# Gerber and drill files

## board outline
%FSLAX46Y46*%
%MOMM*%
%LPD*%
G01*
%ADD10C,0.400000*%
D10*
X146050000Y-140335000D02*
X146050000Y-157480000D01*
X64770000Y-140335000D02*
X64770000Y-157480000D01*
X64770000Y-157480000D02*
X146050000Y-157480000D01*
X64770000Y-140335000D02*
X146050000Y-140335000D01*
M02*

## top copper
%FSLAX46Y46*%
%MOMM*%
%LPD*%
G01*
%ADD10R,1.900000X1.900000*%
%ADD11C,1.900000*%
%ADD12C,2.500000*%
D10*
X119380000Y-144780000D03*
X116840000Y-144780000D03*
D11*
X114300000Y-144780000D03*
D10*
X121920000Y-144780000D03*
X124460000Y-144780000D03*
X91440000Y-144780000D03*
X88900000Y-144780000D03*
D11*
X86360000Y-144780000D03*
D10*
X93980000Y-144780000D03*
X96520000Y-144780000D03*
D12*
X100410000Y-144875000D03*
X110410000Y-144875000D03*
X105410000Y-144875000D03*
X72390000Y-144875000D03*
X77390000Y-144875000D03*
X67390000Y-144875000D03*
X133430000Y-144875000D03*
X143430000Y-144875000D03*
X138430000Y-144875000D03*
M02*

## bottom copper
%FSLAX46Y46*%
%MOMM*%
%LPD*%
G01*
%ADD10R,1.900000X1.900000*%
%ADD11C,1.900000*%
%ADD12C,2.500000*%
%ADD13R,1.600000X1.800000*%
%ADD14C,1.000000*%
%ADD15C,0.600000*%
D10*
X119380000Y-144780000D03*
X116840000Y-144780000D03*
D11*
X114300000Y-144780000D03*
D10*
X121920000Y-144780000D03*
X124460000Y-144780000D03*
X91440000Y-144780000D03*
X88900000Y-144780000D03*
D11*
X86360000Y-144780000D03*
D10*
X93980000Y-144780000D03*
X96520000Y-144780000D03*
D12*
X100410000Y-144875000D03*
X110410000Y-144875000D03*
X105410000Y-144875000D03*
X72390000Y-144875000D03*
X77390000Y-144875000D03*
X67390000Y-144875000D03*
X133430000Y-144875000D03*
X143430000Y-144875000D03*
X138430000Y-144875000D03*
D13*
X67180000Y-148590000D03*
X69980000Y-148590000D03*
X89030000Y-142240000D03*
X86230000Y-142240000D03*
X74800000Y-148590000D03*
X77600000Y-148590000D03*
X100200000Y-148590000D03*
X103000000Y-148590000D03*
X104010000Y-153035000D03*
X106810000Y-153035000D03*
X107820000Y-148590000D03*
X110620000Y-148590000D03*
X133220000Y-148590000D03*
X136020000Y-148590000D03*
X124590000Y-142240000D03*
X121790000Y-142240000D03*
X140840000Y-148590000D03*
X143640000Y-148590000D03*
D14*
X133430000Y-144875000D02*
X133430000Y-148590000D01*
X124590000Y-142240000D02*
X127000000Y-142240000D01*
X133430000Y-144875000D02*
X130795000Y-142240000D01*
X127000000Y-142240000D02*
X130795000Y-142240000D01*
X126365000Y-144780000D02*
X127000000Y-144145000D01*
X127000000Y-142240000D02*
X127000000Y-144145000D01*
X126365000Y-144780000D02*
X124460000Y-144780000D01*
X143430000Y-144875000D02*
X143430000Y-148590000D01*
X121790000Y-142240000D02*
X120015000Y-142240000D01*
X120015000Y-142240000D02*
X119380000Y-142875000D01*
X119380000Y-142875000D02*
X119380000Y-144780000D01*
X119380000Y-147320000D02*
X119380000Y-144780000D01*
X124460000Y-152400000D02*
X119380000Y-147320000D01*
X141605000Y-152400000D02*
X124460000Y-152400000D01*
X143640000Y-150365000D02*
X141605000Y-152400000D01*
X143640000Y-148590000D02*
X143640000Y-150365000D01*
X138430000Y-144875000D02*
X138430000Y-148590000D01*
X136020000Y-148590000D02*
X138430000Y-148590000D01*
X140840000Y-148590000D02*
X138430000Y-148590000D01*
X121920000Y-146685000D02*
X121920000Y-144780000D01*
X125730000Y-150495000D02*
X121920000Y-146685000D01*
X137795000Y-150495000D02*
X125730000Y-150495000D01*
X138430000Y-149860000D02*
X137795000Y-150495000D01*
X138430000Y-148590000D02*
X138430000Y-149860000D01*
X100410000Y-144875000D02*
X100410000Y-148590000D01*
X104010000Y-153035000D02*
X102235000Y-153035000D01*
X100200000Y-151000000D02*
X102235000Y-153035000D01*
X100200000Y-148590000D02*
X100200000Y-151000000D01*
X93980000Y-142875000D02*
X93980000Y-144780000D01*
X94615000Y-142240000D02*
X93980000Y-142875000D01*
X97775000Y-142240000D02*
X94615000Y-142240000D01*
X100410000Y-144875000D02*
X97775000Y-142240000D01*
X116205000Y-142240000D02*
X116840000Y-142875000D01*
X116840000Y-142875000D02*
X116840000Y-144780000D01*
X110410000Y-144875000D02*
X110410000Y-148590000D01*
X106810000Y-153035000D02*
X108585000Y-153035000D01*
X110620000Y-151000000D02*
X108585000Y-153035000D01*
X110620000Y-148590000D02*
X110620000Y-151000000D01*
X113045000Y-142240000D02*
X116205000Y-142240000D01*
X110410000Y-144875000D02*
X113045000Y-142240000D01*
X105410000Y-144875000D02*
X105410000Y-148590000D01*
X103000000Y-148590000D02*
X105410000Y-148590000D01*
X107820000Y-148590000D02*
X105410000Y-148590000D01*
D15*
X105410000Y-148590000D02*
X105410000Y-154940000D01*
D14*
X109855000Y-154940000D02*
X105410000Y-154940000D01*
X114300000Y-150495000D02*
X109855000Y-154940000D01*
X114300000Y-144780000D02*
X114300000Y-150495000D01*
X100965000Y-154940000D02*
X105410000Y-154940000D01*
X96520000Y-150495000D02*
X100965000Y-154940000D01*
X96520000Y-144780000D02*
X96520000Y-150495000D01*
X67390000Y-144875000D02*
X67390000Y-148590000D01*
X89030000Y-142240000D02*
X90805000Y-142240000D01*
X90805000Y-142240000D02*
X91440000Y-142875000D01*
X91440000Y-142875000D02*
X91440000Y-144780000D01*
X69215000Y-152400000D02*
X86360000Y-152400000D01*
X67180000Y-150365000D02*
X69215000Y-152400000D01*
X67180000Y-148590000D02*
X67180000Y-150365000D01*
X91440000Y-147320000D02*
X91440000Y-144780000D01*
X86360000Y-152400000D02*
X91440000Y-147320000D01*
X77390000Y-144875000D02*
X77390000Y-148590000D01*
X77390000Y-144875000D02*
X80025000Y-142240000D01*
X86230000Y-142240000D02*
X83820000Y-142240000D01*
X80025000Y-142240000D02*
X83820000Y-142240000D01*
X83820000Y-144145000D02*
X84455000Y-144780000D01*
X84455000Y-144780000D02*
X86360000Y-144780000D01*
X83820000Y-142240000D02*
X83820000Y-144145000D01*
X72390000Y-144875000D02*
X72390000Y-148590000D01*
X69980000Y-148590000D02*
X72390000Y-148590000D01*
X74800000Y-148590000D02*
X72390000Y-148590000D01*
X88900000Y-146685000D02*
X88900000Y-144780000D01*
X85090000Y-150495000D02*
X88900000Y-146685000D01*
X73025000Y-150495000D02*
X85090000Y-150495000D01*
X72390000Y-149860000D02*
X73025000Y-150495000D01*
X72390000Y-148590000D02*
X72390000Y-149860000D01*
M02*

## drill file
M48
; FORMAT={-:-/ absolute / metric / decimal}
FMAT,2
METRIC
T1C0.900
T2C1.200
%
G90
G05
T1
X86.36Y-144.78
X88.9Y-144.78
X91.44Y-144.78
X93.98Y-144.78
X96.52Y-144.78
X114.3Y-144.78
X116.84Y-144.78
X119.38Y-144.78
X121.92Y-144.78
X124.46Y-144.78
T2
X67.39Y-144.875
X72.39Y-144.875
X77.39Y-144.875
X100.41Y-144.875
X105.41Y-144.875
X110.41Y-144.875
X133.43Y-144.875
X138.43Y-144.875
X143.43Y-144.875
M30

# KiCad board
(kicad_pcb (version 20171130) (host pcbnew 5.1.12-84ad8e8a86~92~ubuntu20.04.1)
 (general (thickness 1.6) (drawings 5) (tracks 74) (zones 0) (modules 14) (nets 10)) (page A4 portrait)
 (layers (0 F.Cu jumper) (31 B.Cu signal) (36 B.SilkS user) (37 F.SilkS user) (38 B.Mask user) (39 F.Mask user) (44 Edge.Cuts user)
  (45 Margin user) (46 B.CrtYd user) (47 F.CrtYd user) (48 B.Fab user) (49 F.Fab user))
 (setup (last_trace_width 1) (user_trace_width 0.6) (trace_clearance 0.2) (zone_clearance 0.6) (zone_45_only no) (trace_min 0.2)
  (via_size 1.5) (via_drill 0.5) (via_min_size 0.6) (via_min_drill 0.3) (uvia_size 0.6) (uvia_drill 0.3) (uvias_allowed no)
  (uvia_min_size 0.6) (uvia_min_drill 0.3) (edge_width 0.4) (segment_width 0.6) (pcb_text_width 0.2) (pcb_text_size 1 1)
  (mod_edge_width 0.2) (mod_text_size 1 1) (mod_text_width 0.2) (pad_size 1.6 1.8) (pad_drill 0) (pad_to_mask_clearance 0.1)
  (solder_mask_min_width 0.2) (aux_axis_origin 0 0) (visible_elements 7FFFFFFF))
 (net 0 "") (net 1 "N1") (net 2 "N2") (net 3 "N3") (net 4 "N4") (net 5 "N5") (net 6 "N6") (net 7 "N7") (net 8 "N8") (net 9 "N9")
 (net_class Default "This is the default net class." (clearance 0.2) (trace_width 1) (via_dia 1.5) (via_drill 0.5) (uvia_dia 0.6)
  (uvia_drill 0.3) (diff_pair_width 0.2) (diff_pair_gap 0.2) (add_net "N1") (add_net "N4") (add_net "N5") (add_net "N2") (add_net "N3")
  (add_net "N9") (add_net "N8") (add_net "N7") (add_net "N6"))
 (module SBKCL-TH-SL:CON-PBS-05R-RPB (layer F.Cu) (at 119.38 144.78)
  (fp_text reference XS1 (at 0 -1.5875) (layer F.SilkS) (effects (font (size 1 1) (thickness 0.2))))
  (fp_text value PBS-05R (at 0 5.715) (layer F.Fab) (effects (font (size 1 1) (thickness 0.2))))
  (pad 3 thru_hole rect (at 0 0) (size 1.9 1.9) (drill 0.9) (layers B.Cu B.Mask) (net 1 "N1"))
  (pad 2 thru_hole rect (at -2.54 0) (size 1.9 1.9) (drill 0.9) (layers B.Cu B.Mask) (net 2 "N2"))
  (pad 1 thru_hole circle (at -5.08 0) (size 1.9 1.9) (drill 0.9) (layers B.Cu B.Mask) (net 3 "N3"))
  (pad 4 thru_hole rect (at 2.54 0) (size 1.9 1.9) (drill 0.9) (layers B.Cu B.Mask) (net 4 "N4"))
  (pad 5 thru_hole rect (at 5.08 0) (size 1.9 1.9) (drill 0.9) (layers B.Cu B.Mask) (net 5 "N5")))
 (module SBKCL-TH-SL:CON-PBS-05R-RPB (layer F.Cu) (at 91.44 144.78)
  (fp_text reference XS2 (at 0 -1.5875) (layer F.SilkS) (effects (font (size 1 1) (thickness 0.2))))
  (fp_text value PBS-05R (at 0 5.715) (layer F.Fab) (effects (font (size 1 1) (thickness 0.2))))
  (pad 3 thru_hole rect (at 0 0) (size 1.9 1.9) (drill 0.9) (layers B.Cu B.Mask) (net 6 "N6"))
  (pad 2 thru_hole rect (at -2.54 0) (size 1.9 1.9) (drill 0.9) (layers B.Cu B.Mask) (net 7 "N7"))
  (pad 1 thru_hole circle (at -5.08 0) (size 1.9 1.9) (drill 0.9) (layers B.Cu B.Mask) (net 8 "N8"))
  (pad 4 thru_hole rect (at 2.54 0) (size 1.9 1.9) (drill 0.9) (layers B.Cu B.Mask) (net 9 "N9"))
  (pad 5 thru_hole rect (at 5.08 0) (size 1.9 1.9) (drill 0.9) (layers B.Cu B.Mask) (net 3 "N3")))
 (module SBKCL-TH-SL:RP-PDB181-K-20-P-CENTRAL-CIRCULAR (layer F.Cu) (at 105.41 144.875 180)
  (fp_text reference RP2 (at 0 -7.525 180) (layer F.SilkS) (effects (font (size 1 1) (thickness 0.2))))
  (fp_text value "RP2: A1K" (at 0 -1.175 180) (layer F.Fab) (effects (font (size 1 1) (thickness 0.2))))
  (pad 3 thru_hole circle (at 5 0 180) (size 2.5 2.5) (drill 1.2) (layers B.Cu B.Mask) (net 9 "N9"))
  (pad 1 thru_hole circle (at -5 0 180) (size 2.5 2.5) (drill 1.2) (layers B.Cu B.Mask) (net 2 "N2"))
  (pad 2 thru_hole circle (at 0 0 180) (size 2.5 2.5) (drill 1.2) (layers B.Cu B.Mask) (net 3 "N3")))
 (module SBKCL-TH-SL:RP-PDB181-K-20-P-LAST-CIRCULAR (layer F.Cu) (at 72.39 144.875 180)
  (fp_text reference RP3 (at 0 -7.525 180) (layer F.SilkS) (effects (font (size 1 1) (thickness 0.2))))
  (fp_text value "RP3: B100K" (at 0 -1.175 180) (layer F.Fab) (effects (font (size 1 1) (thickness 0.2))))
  (pad 2 thru_hole circle (at 0 0 180) (size 2.5 2.5) (drill 1.2) (layers B.Cu B.Mask) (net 7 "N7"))
  (pad 1 thru_hole circle (at -5 0 180) (size 2.5 2.5) (drill 1.2) (layers B.Cu B.Mask) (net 8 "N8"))
  (pad 3 thru_hole circle (at 5 0 180) (size 2.5 2.5) (drill 1.2) (layers B.Cu B.Mask) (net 6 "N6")))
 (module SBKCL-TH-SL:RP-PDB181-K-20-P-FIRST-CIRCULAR (layer F.Cu) (at 138.43 144.875 180)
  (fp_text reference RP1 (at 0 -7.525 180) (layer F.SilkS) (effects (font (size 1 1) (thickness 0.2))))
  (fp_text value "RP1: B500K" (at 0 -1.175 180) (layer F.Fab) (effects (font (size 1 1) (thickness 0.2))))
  (pad 3 thru_hole circle (at 5 0 180) (size 2.5 2.5) (drill 1.2) (layers B.Cu B.Mask) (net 5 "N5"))
  (pad 1 thru_hole circle (at -5 0 180) (size 2.5 2.5) (drill 1.2) (layers B.Cu B.Mask) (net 1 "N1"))
  (pad 2 thru_hole circle (at 0 0 180) (size 2.5 2.5) (drill 1.2) (layers B.Cu B.Mask) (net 4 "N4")))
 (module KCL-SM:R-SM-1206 (layer B.Cu) (at 68.58 148.59)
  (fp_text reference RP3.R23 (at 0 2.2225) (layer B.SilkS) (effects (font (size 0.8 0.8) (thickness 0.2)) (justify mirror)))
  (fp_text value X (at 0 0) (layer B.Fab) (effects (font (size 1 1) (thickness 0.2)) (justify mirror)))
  (pad 1 smd rect (at -1.4 0) (size 1.6 1.8) (layers B.Cu B.Mask) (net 6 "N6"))
  (pad 2 smd rect (at 1.4 0) (size 1.6 1.8) (layers B.Cu B.Mask) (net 7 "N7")))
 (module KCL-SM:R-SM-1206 (layer B.Cu) (at 87.63 142.24 180)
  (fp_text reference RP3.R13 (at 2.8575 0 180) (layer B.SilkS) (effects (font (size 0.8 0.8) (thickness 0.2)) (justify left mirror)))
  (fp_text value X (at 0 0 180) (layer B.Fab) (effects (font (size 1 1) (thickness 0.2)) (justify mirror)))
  (pad 1 smd rect (at -1.4 0 180) (size 1.6 1.8) (layers B.Cu B.Mask) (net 6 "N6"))
  (pad 2 smd rect (at 1.4 0 180) (size 1.6 1.8) (layers B.Cu B.Mask) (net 8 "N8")))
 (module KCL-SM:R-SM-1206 (layer B.Cu) (at 76.2 148.59)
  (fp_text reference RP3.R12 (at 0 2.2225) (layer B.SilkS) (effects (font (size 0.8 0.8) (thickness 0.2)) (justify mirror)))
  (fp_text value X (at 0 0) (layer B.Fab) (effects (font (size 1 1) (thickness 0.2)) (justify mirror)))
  (pad 1 smd rect (at -1.4 0) (size 1.6 1.8) (layers B.Cu B.Mask) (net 7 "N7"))
  (pad 2 smd rect (at 1.4 0) (size 1.6 1.8) (layers B.Cu B.Mask) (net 8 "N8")))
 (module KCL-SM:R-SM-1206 (layer B.Cu) (at 101.6 148.59)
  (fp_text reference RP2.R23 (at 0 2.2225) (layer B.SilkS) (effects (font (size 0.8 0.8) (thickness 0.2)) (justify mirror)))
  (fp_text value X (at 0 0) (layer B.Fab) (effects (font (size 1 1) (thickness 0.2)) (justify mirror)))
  (pad 1 smd rect (at -1.4 0) (size 1.6 1.8) (layers B.Cu B.Mask) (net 9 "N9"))
  (pad 2 smd rect (at 1.4 0) (size 1.6 1.8) (layers B.Cu B.Mask) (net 3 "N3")))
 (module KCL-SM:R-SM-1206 (layer B.Cu) (at 105.41 153.035)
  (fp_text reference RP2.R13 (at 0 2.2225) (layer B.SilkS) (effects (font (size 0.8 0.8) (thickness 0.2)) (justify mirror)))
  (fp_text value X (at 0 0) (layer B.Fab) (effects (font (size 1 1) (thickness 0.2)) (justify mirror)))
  (pad 1 smd rect (at -1.4 0) (size 1.6 1.8) (layers B.Cu B.Mask) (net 9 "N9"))
  (pad 2 smd rect (at 1.4 0) (size 1.6 1.8) (layers B.Cu B.Mask) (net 2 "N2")))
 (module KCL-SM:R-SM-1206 (layer B.Cu) (at 109.22 148.59)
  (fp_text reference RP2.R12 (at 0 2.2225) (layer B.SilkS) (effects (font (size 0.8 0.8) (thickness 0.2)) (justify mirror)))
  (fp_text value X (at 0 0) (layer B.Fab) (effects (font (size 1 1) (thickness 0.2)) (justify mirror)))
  (pad 1 smd rect (at -1.4 0) (size 1.6 1.8) (layers B.Cu B.Mask) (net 3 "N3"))
  (pad 2 smd rect (at 1.4 0) (size 1.6 1.8) (layers B.Cu B.Mask) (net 2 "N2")))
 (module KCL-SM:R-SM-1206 (layer B.Cu) (at 134.62 148.59)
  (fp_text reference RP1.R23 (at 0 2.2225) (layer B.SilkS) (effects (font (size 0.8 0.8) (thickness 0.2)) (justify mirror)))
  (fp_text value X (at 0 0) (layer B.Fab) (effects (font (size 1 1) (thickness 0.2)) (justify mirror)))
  (pad 1 smd rect (at -1.4 0) (size 1.6 1.8) (layers B.Cu B.Mask) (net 5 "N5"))
  (pad 2 smd rect (at 1.4 0) (size 1.6 1.8) (layers B.Cu B.Mask) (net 4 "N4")))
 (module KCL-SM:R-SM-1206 (layer B.Cu) (at 123.19 142.24 180)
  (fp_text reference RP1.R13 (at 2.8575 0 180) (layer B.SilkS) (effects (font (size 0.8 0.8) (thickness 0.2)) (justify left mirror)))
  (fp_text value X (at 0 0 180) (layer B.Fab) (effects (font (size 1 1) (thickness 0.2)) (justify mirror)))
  (pad 1 smd rect (at -1.4 0 180) (size 1.6 1.8) (layers B.Cu B.Mask) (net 5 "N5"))
  (pad 2 smd rect (at 1.4 0 180) (size 1.6 1.8) (layers B.Cu B.Mask) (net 1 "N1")))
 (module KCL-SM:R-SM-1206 (layer B.Cu) (at 142.24 148.59)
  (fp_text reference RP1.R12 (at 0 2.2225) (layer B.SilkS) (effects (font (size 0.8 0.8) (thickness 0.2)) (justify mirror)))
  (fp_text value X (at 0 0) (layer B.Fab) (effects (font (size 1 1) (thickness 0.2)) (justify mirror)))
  (pad 1 smd rect (at -1.4 0) (size 1.6 1.8) (layers B.Cu B.Mask) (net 4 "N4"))
  (pad 2 smd rect (at 1.4 0) (size 1.6 1.8) (layers B.Cu B.Mask) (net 1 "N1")))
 (gr_line (start 146.05 140.335) (end 146.05 157.48) (layer Edge.Cuts) (width 0.4))
 (gr_line (start 64.77 140.335) (end 64.77 157.48) (layer Edge.Cuts) (width 0.4))
 (gr_line (start 64.77 157.48) (end 146.05 157.48) (layer Edge.Cuts) (width 0.4))
 (gr_line (start 64.77 140.335) (end 146.05 140.335) (layer Edge.Cuts) (width 0.4))
 (segment (start 133.43 144.875) (end 133.43 148.59) (width 1) (layer B.Cu) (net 5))
 (segment (start 124.59 142.24) (end 127 142.24) (width 1) (layer B.Cu) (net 5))
 (segment (start 133.43 144.875) (end 130.795 142.24) (width 1) (layer B.Cu) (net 5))
 (segment (start 127 142.24) (end 130.795 142.24) (width 1) (layer B.Cu) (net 5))
 (segment (start 126.365 144.78) (end 127 144.145) (width 1) (layer B.Cu) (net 5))
 (segment (start 127 142.24) (end 127 144.145) (width 1) (layer B.Cu) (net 5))
 (segment (start 126.365 144.78) (end 124.46 144.78) (width 1) (layer B.Cu) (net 5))
 (segment (start 143.43 144.875) (end 143.43 148.59) (width 1) (layer B.Cu) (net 1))
 (segment (start 121.79 142.24) (end 120.015 142.24) (width 1) (layer B.Cu) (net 1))
 (segment (start 120.015 142.24) (end 119.38 142.875) (width 1) (layer B.Cu) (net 1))
 (segment (start 119.38 142.875) (end 119.38 144.78) (width 1) (layer B.Cu) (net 1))
 (segment (start 119.38 147.32) (end 119.38 144.78) (width 1) (layer B.Cu) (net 1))
 (segment (start 124.46 152.4) (end 119.38 147.32) (width 1) (layer B.Cu) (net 1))
 (segment (start 141.605 152.4) (end 124.46 152.4) (width 1) (layer B.Cu) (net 1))
 (segment (start 143.64 150.365) (end 141.605 152.4) (width 1) (layer B.Cu) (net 1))
 (segment (start 143.64 148.59) (end 143.64 150.365) (width 1) (layer B.Cu) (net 1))
 (segment (start 138.43 144.875) (end 138.43 148.59) (width 1) (layer B.Cu) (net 4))
 (segment (start 136.02 148.59) (end 138.43 148.59) (width 1) (layer B.Cu) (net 4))
 (segment (start 140.84 148.59) (end 138.43 148.59) (width 1) (layer B.Cu) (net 4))
 (segment (start 121.92 146.685) (end 121.92 144.78) (width 1) (layer B.Cu) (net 4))
 (segment (start 125.73 150.495) (end 121.92 146.685) (width 1) (layer B.Cu) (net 4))
 (segment (start 137.795 150.495) (end 125.73 150.495) (width 1) (layer B.Cu) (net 4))
 (segment (start 138.43 149.86) (end 137.795 150.495) (width 1) (layer B.Cu) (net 4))
 (segment (start 138.43 148.59) (end 138.43 149.86) (width 1) (layer B.Cu) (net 4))
 (segment (start 100.41 144.875) (end 100.41 148.59) (width 1) (layer B.Cu) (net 9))
 (segment (start 104.01 153.035) (end 102.235 153.035) (width 1) (layer B.Cu) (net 9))
 (segment (start 100.2 151) (end 102.235 153.035) (width 1) (layer B.Cu) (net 9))
 (segment (start 100.2 148.59) (end 100.2 151) (width 1) (layer B.Cu) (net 9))
 (segment (start 93.98 142.875) (end 93.98 144.78) (width 1) (layer B.Cu) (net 9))
 (segment (start 94.615 142.24) (end 93.98 142.875) (width 1) (layer B.Cu) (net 9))
 (segment (start 97.775 142.24) (end 94.615 142.24) (width 1) (layer B.Cu) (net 9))
 (segment (start 100.41 144.875) (end 97.775 142.24) (width 1) (layer B.Cu) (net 9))
 (segment (start 116.205 142.24) (end 116.84 142.875) (width 1) (layer B.Cu) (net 2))
 (segment (start 116.84 142.875) (end 116.84 144.78) (width 1) (layer B.Cu) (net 2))
 (segment (start 110.41 144.875) (end 110.41 148.59) (width 1) (layer B.Cu) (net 2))
 (segment (start 106.81 153.035) (end 108.585 153.035) (width 1) (layer B.Cu) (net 2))
 (segment (start 110.62 151) (end 108.585 153.035) (width 1) (layer B.Cu) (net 2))
 (segment (start 110.62 148.59) (end 110.62 151) (width 1) (layer B.Cu) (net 2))
 (segment (start 113.045 142.24) (end 116.205 142.24) (width 1) (layer B.Cu) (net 2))
 (segment (start 110.41 144.875) (end 113.045 142.24) (width 1) (layer B.Cu) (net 2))
 (segment (start 105.41 144.875) (end 105.41 148.59) (width 1) (layer B.Cu) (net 3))
 (segment (start 103 148.59) (end 105.41 148.59) (width 1) (layer B.Cu) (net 3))
 (segment (start 107.82 148.59) (end 105.41 148.59) (width 1) (layer B.Cu) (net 3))
 (segment (start 105.41 148.59) (end 105.41 154.94) (width 0.6) (layer B.Cu) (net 3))
 (segment (start 109.855 154.94) (end 105.41 154.94) (width 1) (layer B.Cu) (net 3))
 (segment (start 114.3 150.495) (end 109.855 154.94) (width 1) (layer B.Cu) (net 3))
 (segment (start 114.3 144.78) (end 114.3 150.495) (width 1) (layer B.Cu) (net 3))
 (segment (start 100.965 154.94) (end 105.41 154.94) (width 1) (layer B.Cu) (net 3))
 (segment (start 96.52 150.495) (end 100.965 154.94) (width 1) (layer B.Cu) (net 3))
 (segment (start 96.52 144.78) (end 96.52 150.495) (width 1) (layer B.Cu) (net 3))
 (segment (start 67.39 144.875) (end 67.39 148.59) (width 1) (layer B.Cu) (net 6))
 (segment (start 89.03 142.24) (end 90.805 142.24) (width 1) (layer B.Cu) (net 6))
 (segment (start 90.805 142.24) (end 91.44 142.875) (width 1) (layer B.Cu) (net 6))
 (segment (start 91.44 142.875) (end 91.44 144.78) (width 1) (layer B.Cu) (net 6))
 (segment (start 69.215 152.4) (end 86.36 152.4) (width 1) (layer B.Cu) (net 6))
 (segment (start 67.18 150.365) (end 69.215 152.4) (width 1) (layer B.Cu) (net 6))
 (segment (start 67.18 148.59) (end 67.18 150.365) (width 1) (layer B.Cu) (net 6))
 (segment (start 91.44 147.32) (end 91.44 144.78) (width 1) (layer B.Cu) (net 6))
 (segment (start 86.36 152.4) (end 91.44 147.32) (width 1) (layer B.Cu) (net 6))
 (segment (start 77.39 144.875) (end 77.39 148.59) (width 1) (layer B.Cu) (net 8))
 (segment (start 77.39 144.875) (end 80.025 142.24) (width 1) (layer B.Cu) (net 8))
 (segment (start 86.23 142.24) (end 83.82 142.24) (width 1) (layer B.Cu) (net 8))
 (segment (start 80.025 142.24) (end 83.82 142.24) (width 1) (layer B.Cu) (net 8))
 (segment (start 83.82 144.145) (end 84.455 144.78) (width 1) (layer B.Cu) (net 8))
 (segment (start 84.455 144.78) (end 86.36 144.78) (width 1) (layer B.Cu) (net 8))
 (segment (start 83.82 142.24) (end 83.82 144.145) (width 1) (layer B.Cu) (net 8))
 (segment (start 72.39 144.875) (end 72.39 148.59) (width 1) (layer B.Cu) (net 7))
 (segment (start 69.98 148.59) (end 72.39 148.59) (width 1) (layer B.Cu) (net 7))
 (segment (start 74.8 148.59) (end 72.39 148.59) (width 1) (layer B.Cu) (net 7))
 (segment (start 88.9 146.685) (end 88.9 144.78) (width 1) (layer B.Cu) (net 7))
 (segment (start 85.09 150.495) (end 88.9 146.685) (width 1) (layer B.Cu) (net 7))
 (segment (start 73.025 150.495) (end 85.09 150.495) (width 1) (layer B.Cu) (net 7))
 (segment (start 72.39 149.86) (end 73.025 150.495) (width 1) (layer B.Cu) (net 7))
 (segment (start 72.39 148.59) (end 72.39 149.86) (width 1) (layer B.Cu) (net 7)))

